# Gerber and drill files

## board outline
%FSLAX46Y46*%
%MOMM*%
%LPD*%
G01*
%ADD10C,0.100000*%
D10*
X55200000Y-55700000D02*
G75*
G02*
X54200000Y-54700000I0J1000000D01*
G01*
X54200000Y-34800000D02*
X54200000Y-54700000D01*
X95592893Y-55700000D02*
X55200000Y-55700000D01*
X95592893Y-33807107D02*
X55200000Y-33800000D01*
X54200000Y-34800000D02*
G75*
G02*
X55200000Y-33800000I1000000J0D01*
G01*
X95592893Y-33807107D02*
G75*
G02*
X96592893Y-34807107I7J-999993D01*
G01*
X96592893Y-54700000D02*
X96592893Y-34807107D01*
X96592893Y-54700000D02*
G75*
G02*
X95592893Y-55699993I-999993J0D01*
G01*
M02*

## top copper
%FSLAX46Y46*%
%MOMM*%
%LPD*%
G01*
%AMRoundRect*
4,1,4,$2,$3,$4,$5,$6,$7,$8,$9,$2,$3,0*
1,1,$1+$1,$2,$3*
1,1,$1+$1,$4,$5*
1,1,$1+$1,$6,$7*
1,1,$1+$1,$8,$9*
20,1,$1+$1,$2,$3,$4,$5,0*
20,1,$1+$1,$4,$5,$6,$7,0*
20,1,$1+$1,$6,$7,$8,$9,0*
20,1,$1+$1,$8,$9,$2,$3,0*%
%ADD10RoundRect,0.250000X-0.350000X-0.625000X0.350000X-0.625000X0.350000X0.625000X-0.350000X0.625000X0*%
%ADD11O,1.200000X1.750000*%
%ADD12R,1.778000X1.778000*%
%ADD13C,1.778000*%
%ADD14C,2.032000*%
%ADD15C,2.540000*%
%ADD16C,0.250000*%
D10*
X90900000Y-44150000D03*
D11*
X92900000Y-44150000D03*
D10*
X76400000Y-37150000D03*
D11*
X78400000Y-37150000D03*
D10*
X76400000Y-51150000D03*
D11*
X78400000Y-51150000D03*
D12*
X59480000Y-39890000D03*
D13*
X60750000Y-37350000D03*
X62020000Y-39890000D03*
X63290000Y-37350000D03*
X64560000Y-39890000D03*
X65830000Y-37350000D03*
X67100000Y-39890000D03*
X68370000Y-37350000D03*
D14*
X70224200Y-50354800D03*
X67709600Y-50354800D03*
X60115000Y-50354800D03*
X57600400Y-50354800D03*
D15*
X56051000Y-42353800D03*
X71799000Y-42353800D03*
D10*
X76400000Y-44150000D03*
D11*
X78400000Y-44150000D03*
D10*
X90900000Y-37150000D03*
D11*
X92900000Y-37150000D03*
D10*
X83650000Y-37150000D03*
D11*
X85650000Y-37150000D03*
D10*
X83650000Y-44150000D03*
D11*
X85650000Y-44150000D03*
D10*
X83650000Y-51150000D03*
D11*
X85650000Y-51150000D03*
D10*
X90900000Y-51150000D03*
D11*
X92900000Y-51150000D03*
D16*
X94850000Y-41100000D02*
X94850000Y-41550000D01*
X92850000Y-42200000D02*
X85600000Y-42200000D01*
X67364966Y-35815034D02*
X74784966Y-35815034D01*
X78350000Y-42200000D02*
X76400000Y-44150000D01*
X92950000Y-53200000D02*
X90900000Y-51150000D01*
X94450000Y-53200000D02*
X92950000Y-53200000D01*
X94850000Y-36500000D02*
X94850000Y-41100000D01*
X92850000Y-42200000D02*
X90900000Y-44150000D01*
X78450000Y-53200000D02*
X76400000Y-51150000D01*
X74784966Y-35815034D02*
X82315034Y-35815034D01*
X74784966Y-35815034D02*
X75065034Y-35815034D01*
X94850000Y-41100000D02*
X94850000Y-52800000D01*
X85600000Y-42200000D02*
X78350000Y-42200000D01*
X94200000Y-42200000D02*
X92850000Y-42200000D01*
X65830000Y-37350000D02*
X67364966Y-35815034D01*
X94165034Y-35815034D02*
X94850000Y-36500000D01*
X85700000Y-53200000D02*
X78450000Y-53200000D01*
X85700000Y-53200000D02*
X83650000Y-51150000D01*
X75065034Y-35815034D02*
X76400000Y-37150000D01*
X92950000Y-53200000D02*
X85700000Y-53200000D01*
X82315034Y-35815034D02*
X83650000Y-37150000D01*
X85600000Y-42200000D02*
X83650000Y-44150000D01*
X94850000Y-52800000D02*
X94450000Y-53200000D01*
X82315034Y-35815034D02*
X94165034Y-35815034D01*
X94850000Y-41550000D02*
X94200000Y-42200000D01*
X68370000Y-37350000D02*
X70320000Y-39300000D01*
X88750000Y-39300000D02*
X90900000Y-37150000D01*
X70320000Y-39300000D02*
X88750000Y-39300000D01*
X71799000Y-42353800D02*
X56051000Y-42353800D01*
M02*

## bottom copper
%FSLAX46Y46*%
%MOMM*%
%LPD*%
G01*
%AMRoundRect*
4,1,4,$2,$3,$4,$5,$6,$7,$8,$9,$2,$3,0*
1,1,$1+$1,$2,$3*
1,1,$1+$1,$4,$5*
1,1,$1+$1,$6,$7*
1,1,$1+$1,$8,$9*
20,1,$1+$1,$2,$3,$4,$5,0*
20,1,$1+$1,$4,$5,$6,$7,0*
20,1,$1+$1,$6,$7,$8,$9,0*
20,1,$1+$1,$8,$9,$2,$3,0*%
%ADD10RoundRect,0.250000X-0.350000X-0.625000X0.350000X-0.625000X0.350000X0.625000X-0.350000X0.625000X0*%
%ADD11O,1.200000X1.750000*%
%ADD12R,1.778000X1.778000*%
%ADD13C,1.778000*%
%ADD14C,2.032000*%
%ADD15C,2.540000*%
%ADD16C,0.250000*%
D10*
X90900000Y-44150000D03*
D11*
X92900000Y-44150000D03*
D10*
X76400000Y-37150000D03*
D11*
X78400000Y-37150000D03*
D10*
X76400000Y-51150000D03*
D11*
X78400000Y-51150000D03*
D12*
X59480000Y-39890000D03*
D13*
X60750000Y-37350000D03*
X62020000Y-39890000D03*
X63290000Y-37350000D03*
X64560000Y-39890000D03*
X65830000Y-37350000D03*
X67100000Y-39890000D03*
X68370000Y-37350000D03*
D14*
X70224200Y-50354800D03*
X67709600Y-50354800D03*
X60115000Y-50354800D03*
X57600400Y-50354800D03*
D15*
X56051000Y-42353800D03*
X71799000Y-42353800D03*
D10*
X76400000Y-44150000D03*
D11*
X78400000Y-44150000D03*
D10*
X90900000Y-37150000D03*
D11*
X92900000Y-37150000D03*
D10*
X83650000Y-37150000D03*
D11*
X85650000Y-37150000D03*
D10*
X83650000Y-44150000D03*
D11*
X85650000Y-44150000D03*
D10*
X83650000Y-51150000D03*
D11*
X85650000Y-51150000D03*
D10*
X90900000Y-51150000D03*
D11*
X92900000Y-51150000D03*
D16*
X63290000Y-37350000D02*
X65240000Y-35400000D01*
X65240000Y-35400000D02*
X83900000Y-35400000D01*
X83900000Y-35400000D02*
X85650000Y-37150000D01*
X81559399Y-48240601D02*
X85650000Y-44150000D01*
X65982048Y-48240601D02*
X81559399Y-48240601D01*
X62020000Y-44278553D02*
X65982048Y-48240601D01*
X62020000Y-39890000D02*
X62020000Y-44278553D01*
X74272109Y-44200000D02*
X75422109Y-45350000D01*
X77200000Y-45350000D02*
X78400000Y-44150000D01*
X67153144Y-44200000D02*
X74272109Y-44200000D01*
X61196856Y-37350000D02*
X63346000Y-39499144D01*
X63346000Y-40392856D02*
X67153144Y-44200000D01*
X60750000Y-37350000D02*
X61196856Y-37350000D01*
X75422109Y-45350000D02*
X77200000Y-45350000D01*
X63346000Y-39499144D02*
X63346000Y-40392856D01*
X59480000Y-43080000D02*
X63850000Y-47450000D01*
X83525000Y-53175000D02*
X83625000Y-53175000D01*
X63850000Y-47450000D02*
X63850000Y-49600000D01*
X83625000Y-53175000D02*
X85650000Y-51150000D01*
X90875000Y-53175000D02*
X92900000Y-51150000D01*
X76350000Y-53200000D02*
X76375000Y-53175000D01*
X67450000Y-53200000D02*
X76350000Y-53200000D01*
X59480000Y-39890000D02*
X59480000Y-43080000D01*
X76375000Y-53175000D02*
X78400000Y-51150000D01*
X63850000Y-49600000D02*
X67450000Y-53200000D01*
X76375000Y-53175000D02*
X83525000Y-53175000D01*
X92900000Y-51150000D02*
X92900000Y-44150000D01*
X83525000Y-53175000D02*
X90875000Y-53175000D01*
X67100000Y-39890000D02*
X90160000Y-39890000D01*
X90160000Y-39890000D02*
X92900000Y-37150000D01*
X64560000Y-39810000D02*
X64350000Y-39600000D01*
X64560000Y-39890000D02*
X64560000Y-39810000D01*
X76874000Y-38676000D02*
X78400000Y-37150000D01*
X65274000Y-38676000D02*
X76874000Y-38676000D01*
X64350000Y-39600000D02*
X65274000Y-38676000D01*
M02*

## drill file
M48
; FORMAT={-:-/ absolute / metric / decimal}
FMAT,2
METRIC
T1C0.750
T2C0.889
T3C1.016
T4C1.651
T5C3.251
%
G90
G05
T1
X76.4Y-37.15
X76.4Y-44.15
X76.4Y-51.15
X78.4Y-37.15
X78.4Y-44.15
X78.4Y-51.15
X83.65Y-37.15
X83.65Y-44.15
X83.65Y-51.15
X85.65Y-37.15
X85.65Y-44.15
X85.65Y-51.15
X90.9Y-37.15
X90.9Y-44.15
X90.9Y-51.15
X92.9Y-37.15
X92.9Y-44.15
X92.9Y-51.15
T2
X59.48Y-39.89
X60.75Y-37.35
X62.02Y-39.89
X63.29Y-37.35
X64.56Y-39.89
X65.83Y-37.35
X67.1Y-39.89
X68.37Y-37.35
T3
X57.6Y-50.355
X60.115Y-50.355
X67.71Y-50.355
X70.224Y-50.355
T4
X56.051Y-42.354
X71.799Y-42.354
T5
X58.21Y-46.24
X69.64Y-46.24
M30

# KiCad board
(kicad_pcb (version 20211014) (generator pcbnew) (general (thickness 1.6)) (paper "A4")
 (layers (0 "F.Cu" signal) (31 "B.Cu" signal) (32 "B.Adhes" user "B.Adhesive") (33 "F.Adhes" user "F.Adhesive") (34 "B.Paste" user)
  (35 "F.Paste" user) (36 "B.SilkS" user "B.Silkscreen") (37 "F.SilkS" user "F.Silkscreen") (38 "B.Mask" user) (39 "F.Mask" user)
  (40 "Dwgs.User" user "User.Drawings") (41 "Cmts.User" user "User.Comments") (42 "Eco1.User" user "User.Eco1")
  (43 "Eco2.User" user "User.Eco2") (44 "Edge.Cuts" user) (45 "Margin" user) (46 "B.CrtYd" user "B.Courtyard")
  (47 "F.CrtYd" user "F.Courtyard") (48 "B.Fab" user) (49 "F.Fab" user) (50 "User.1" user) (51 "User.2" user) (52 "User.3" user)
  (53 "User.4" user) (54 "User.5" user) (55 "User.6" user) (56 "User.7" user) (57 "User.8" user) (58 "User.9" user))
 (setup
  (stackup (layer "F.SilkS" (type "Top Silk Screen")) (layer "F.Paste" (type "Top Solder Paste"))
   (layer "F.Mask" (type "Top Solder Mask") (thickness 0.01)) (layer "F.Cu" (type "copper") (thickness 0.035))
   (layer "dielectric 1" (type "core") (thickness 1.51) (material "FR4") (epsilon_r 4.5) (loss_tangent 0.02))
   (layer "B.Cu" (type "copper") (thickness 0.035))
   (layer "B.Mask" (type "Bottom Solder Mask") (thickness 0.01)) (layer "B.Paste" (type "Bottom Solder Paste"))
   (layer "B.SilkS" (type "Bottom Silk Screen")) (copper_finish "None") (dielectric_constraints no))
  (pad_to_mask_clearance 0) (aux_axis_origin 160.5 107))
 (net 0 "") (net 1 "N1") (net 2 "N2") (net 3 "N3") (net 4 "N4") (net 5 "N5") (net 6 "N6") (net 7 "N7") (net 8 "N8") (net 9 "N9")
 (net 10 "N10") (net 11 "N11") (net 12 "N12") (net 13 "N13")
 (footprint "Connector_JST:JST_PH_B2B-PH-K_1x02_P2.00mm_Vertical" (layer "F.Cu") (at 90.9 44.15)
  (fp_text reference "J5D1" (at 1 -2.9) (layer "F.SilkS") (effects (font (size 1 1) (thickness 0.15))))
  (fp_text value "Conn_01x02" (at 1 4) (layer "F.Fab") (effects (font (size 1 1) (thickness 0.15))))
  (pad "1" thru_hole roundrect (at 0 0) (size 1.2 1.75) (drill 0.75) (layers *.Cu *.Mask) (roundrect_rratio 0.208333) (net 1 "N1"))
  (pad "2" thru_hole oval (at 2 0) (size 1.2 1.75) (drill 0.75) (layers *.Cu *.Mask) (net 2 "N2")))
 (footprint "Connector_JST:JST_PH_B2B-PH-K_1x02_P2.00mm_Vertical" (layer "F.Cu") (at 76.4 37.15)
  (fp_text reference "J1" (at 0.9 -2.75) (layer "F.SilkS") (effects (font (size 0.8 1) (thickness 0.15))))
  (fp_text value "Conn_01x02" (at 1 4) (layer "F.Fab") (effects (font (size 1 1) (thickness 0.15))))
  (pad "1" thru_hole roundrect (at 0 0) (size 1.2 1.75) (drill 0.75) (layers *.Cu *.Mask) (roundrect_rratio 0.208333) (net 1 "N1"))
  (pad "2" thru_hole oval (at 2 0) (size 1.2 1.75) (drill 0.75) (layers *.Cu *.Mask) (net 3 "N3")))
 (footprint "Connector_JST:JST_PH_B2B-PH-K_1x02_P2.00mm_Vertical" (layer "F.Cu") (at 76.4 51.15)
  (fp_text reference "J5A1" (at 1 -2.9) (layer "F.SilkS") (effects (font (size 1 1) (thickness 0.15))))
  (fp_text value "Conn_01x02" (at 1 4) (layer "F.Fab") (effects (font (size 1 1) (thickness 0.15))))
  (pad "1" thru_hole roundrect (at 0 0) (size 1.2 1.75) (drill 0.75) (layers *.Cu *.Mask) (roundrect_rratio 0.208333) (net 1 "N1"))
  (pad "2" thru_hole oval (at 2 0) (size 1.2 1.75) (drill 0.75) (layers *.Cu *.Mask) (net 2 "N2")))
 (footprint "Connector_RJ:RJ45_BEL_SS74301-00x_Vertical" (layer "F.Cu") (at 59.48 39.89)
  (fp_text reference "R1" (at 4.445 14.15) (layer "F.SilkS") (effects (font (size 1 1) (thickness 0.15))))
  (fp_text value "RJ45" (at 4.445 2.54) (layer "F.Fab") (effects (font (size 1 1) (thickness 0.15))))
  (pad "" np_thru_hole circle (at -1.27 6.35) (size 3.2512 3.2512) (drill 3.2512) (layers *.Cu *.Mask))
  (pad "" np_thru_hole circle (at 10.16 6.35) (size 3.2512 3.2512) (drill 3.2512) (layers *.Cu *.Mask))
  (pad "1" thru_hole rect (at 0 0) (size 1.778 1.778) (drill 0.889) (layers *.Cu *.Mask) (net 2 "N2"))
  (pad "2" thru_hole circle (at 1.27 -2.54) (size 1.778 1.778) (drill 0.889) (layers *.Cu *.Mask) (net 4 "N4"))
  (pad "3" thru_hole circle (at 2.54 0) (size 1.778 1.778) (drill 0.889) (layers *.Cu *.Mask) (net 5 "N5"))
  (pad "4" thru_hole circle (at 3.81 -2.54) (size 1.778 1.778) (drill 0.889) (layers *.Cu *.Mask) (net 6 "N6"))
  (pad "5" thru_hole circle (at 5.08 0) (size 1.778 1.778) (drill 0.889) (layers *.Cu *.Mask) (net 3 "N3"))
  (pad "6" thru_hole circle (at 6.35 -2.54) (size 1.778 1.778) (drill 0.889) (layers *.Cu *.Mask) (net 1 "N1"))
  (pad "7" thru_hole circle (at 7.62 0) (size 1.778 1.778) (drill 0.889) (layers *.Cu *.Mask) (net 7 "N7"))
  (pad "8" thru_hole circle (at 8.89 -2.54) (size 1.778 1.778) (drill 0.889) (layers *.Cu *.Mask) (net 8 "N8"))
  (pad "9" thru_hole circle (at 10.7442 10.4648) (size 2.032 2.032) (drill 1.016) (layers *.Cu *.Mask) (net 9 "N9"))
  (pad "10" thru_hole circle (at 8.2296 10.4648) (size 2.032 2.032) (drill 1.016) (layers *.Cu *.Mask) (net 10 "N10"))
  (pad "11" thru_hole circle (at 0.635 10.4648) (size 2.032 2.032) (drill 1.016) (layers *.Cu *.Mask) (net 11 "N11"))
  (pad "12" thru_hole circle (at -1.8796 10.4648) (size 2.032 2.032) (drill 1.016) (layers *.Cu *.Mask) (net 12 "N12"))
  (pad "SH" thru_hole circle (at -3.429 2.4638) (size 2.54 2.54) (drill 1.651) (layers *.Cu *.Mask) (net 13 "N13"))
  (pad "SH" thru_hole circle (at 12.319 2.4638) (size 2.54 2.54) (drill 1.651) (layers *.Cu *.Mask) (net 13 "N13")))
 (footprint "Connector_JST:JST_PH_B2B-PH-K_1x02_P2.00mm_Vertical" (layer "F.Cu") (at 76.4 44.15)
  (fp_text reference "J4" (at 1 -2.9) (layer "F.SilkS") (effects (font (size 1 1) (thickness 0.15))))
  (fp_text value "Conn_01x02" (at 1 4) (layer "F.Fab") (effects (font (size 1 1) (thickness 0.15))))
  (pad "1" thru_hole roundrect (at 0 0) (size 1.2 1.75) (drill 0.75) (layers *.Cu *.Mask) (roundrect_rratio 0.208333) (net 1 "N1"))
  (pad "2" thru_hole oval (at 2 0) (size 1.2 1.75) (drill 0.75) (layers *.Cu *.Mask) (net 4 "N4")))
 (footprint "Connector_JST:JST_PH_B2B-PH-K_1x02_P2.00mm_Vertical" (layer "F.Cu") (at 90.9 37.15)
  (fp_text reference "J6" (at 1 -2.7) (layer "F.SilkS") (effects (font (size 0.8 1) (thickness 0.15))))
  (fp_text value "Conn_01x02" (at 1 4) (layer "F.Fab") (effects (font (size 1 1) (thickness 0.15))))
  (pad "1" thru_hole roundrect (at 0 0) (size 1.2 1.75) (drill 0.75) (layers *.Cu *.Mask) (roundrect_rratio 0.208333) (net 8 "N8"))
  (pad "2" thru_hole oval (at 2 0) (size 1.2 1.75) (drill 0.75) (layers *.Cu *.Mask) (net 7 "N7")))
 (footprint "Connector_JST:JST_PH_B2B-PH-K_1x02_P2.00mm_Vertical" (layer "F.Cu") (at 83.65 37.15)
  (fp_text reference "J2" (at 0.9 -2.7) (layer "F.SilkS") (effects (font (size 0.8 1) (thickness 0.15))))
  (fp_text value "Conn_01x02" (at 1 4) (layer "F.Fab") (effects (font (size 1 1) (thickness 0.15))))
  (pad "1" thru_hole roundrect (at 0 0) (size 1.2 1.75) (drill 0.75) (layers *.Cu *.Mask) (roundrect_rratio 0.208333) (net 1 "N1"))
  (pad "2" thru_hole oval (at 2 0) (size 1.2 1.75) (drill 0.75) (layers *.Cu *.Mask) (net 6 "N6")))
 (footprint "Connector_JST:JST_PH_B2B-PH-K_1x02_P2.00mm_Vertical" (layer "F.Cu") (at 83.65 44.15)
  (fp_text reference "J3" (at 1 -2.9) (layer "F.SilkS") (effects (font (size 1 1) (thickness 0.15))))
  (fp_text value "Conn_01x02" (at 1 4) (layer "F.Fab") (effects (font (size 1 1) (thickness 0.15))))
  (pad "1" thru_hole roundrect (at 0 0) (size 1.2 1.75) (drill 0.75) (layers *.Cu *.Mask) (roundrect_rratio 0.208333) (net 1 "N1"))
  (pad "2" thru_hole oval (at 2 0) (size 1.2 1.75) (drill 0.75) (layers *.Cu *.Mask) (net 5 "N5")))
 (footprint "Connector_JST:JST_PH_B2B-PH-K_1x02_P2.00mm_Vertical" (layer "F.Cu") (at 83.65 51.15)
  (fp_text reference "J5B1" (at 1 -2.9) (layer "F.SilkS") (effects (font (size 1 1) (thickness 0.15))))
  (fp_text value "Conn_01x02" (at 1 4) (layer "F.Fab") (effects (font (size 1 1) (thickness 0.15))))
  (pad "1" thru_hole roundrect (at 0 0) (size 1.2 1.75) (drill 0.75) (layers *.Cu *.Mask) (roundrect_rratio 0.208333) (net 1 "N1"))
  (pad "2" thru_hole oval (at 2 0) (size 1.2 1.75) (drill 0.75) (layers *.Cu *.Mask) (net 2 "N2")))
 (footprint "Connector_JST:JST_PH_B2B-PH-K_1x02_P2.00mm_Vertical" (layer "F.Cu") (at 90.9 51.15)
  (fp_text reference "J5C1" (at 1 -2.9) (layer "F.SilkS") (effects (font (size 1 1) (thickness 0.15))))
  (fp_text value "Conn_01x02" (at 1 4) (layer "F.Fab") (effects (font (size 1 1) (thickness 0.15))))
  (pad "1" thru_hole roundrect (at 0 0) (size 1.2 1.75) (drill 0.75) (layers *.Cu *.Mask) (roundrect_rratio 0.208333) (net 1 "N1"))
  (pad "2" thru_hole oval (at 2 0) (size 1.2 1.75) (drill 0.75) (layers *.Cu *.Mask) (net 2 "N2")))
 (gr_arc (start 55.2 55.7) (mid 54.492893 55.407107) (end 54.2 54.7) (layer "Edge.Cuts") (width 0.1))
 (gr_line (start 54.2 34.8) (end 54.2 54.7) (layer "Edge.Cuts") (width 0.1))
 (gr_line (start 95.592893 55.7) (end 55.2 55.7) (layer "Edge.Cuts") (width 0.1))
 (gr_line (start 95.592893 33.807107) (end 55.2 33.8) (layer "Edge.Cuts") (width 0.1))
 (gr_arc (start 54.2 34.8) (mid 54.492893 34.092893) (end 55.2 33.8) (layer "Edge.Cuts") (width 0.1))
 (gr_arc (start 95.592893 33.807107) (mid 96.3 34.1) (end 96.592893 34.807107) (layer "Edge.Cuts") (width 0.1))
 (gr_line (start 96.592893 54.7) (end 96.592893 34.807107) (layer "Edge.Cuts") (width 0.1))
 (gr_arc (start 96.592893 54.7) (mid 96.3 55.407107) (end 95.592893 55.7) (layer "Edge.Cuts") (width 0.1))
 (segment (start 94.85 41.1) (end 94.85 41.55) (width 0.25) (layer "F.Cu") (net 1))
 (segment (start 92.85 42.2) (end 85.6 42.2) (width 0.25) (layer "F.Cu") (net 1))
 (segment (start 67.364966 35.815034) (end 74.784966 35.815034) (width 0.25) (layer "F.Cu") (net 1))
 (segment (start 78.35 42.2) (end 76.4 44.15) (width 0.25) (layer "F.Cu") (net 1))
 (segment (start 92.95 53.2) (end 90.9 51.15) (width 0.25) (layer "F.Cu") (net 1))
 (segment (start 94.45 53.2) (end 92.95 53.2) (width 0.25) (layer "F.Cu") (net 1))
 (segment (start 94.85 36.5) (end 94.85 41.1) (width 0.25) (layer "F.Cu") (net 1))
 (segment (start 92.85 42.2) (end 90.9 44.15) (width 0.25) (layer "F.Cu") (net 1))
 (segment (start 78.45 53.2) (end 76.4 51.15) (width 0.25) (layer "F.Cu") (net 1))
 (segment (start 74.784966 35.815034) (end 82.315034 35.815034) (width 0.25) (layer "F.Cu") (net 1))
 (segment (start 74.784966 35.815034) (end 75.065034 35.815034) (width 0.25) (layer "F.Cu") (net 1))
 (segment (start 94.85 41.1) (end 94.85 52.8) (width 0.25) (layer "F.Cu") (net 1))
 (segment (start 85.6 42.2) (end 78.35 42.2) (width 0.25) (layer "F.Cu") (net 1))
 (segment (start 94.2 42.2) (end 92.85 42.2) (width 0.25) (layer "F.Cu") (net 1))
 (segment (start 65.83 37.35) (end 67.364966 35.815034) (width 0.25) (layer "F.Cu") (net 1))
 (segment (start 94.165034 35.815034) (end 94.85 36.5) (width 0.25) (layer "F.Cu") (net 1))
 (segment (start 85.7 53.2) (end 78.45 53.2) (width 0.25) (layer "F.Cu") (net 1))
 (segment (start 85.7 53.2) (end 83.65 51.15) (width 0.25) (layer "F.Cu") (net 1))
 (segment (start 75.065034 35.815034) (end 76.4 37.15) (width 0.25) (layer "F.Cu") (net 1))
 (segment (start 92.95 53.2) (end 85.7 53.2) (width 0.25) (layer "F.Cu") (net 1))
 (segment (start 82.315034 35.815034) (end 83.65 37.15) (width 0.25) (layer "F.Cu") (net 1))
 (segment (start 85.6 42.2) (end 83.65 44.15) (width 0.25) (layer "F.Cu") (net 1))
 (segment (start 94.85 52.8) (end 94.45 53.2) (width 0.25) (layer "F.Cu") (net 1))
 (segment (start 82.315034 35.815034) (end 94.165034 35.815034) (width 0.25) (layer "F.Cu") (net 1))
 (segment (start 94.85 41.55) (end 94.2 42.2) (width 0.25) (layer "F.Cu") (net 1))
 (segment (start 63.29 37.35) (end 65.24 35.4) (width 0.25) (layer "B.Cu") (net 6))
 (segment (start 65.24 35.4) (end 83.9 35.4) (width 0.25) (layer "B.Cu") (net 6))
 (segment (start 83.9 35.4) (end 85.65 37.15) (width 0.25) (layer "B.Cu") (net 6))
 (segment (start 81.559399 48.240601) (end 85.65 44.15) (width 0.25) (layer "B.Cu") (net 5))
 (segment (start 65.982048 48.240601) (end 81.559399 48.240601) (width 0.25) (layer "B.Cu") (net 5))
 (segment (start 62.02 44.278553) (end 65.982048 48.240601) (width 0.25) (layer "B.Cu") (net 5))
 (segment (start 62.02 39.89) (end 62.02 44.278553) (width 0.25) (layer "B.Cu") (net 5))
 (segment (start 74.272109 44.2) (end 75.422109 45.35) (width 0.25) (layer "B.Cu") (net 4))
 (segment (start 77.2 45.35) (end 78.4 44.15) (width 0.25) (layer "B.Cu") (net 4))
 (segment (start 67.153144 44.2) (end 74.272109 44.2) (width 0.25) (layer "B.Cu") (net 4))
 (segment (start 61.196856 37.35) (end 63.346 39.499144) (width 0.25) (layer "B.Cu") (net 4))
 (segment (start 63.346 40.392856) (end 67.153144 44.2) (width 0.25) (layer "B.Cu") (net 4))
 (segment (start 60.75 37.35) (end 61.196856 37.35) (width 0.25) (layer "B.Cu") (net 4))
 (segment (start 75.422109 45.35) (end 77.2 45.35) (width 0.25) (layer "B.Cu") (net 4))
 (segment (start 63.346 39.499144) (end 63.346 40.392856) (width 0.25) (layer "B.Cu") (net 4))
 (segment (start 59.48 43.08) (end 63.85 47.45) (width 0.25) (layer "B.Cu") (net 2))
 (segment (start 83.525 53.175) (end 83.625 53.175) (width 0.25) (layer "B.Cu") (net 2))
 (segment (start 63.85 47.45) (end 63.85 49.6) (width 0.25) (layer "B.Cu") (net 2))
 (segment (start 83.625 53.175) (end 85.65 51.15) (width 0.25) (layer "B.Cu") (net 2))
 (segment (start 90.875 53.175) (end 92.9 51.15) (width 0.25) (layer "B.Cu") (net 2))
 (segment (start 76.35 53.2) (end 76.375 53.175) (width 0.25) (layer "B.Cu") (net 2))
 (segment (start 67.45 53.2) (end 76.35 53.2) (width 0.25) (layer "B.Cu") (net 2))
 (segment (start 59.48 39.89) (end 59.48 43.08) (width 0.25) (layer "B.Cu") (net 2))
 (segment (start 76.375 53.175) (end 78.4 51.15) (width 0.25) (layer "B.Cu") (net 2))
 (segment (start 63.85 49.6) (end 67.45 53.2) (width 0.25) (layer "B.Cu") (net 2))
 (segment (start 76.375 53.175) (end 83.525 53.175) (width 0.25) (layer "B.Cu") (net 2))
 (segment (start 92.9 51.15) (end 92.9 44.15) (width 0.25) (layer "B.Cu") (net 2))
 (segment (start 83.525 53.175) (end 90.875 53.175) (width 0.25) (layer "B.Cu") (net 2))
 (segment (start 68.37 37.35) (end 70.32 39.3) (width 0.25) (layer "F.Cu") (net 8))
 (segment (start 88.75 39.3) (end 90.9 37.15) (width 0.25) (layer "F.Cu") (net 8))
 (segment (start 70.32 39.3) (end 88.75 39.3) (width 0.25) (layer "F.Cu") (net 8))
 (segment (start 67.1 39.89) (end 90.16 39.89) (width 0.25) (layer "B.Cu") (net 7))
 (segment (start 90.16 39.89) (end 92.9 37.15) (width 0.25) (layer "B.Cu") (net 7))
 (segment (start 71.799 42.3538) (end 56.051 42.3538) (width 0.25) (layer "F.Cu") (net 13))
 (segment (start 64.56 39.81) (end 64.35 39.6) (width 0.25) (layer "B.Cu") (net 3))
 (segment (start 64.56 39.89) (end 64.56 39.81) (width 0.25) (layer "B.Cu") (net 3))
 (segment (start 76.874 38.676) (end 78.4 37.15) (width 0.25) (layer "B.Cu") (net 3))
 (segment (start 65.274 38.676) (end 76.874 38.676) (width 0.25) (layer "B.Cu") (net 3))
 (segment (start 64.35 39.6) (end 65.274 38.676) (width 0.25) (layer "B.Cu") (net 3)))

